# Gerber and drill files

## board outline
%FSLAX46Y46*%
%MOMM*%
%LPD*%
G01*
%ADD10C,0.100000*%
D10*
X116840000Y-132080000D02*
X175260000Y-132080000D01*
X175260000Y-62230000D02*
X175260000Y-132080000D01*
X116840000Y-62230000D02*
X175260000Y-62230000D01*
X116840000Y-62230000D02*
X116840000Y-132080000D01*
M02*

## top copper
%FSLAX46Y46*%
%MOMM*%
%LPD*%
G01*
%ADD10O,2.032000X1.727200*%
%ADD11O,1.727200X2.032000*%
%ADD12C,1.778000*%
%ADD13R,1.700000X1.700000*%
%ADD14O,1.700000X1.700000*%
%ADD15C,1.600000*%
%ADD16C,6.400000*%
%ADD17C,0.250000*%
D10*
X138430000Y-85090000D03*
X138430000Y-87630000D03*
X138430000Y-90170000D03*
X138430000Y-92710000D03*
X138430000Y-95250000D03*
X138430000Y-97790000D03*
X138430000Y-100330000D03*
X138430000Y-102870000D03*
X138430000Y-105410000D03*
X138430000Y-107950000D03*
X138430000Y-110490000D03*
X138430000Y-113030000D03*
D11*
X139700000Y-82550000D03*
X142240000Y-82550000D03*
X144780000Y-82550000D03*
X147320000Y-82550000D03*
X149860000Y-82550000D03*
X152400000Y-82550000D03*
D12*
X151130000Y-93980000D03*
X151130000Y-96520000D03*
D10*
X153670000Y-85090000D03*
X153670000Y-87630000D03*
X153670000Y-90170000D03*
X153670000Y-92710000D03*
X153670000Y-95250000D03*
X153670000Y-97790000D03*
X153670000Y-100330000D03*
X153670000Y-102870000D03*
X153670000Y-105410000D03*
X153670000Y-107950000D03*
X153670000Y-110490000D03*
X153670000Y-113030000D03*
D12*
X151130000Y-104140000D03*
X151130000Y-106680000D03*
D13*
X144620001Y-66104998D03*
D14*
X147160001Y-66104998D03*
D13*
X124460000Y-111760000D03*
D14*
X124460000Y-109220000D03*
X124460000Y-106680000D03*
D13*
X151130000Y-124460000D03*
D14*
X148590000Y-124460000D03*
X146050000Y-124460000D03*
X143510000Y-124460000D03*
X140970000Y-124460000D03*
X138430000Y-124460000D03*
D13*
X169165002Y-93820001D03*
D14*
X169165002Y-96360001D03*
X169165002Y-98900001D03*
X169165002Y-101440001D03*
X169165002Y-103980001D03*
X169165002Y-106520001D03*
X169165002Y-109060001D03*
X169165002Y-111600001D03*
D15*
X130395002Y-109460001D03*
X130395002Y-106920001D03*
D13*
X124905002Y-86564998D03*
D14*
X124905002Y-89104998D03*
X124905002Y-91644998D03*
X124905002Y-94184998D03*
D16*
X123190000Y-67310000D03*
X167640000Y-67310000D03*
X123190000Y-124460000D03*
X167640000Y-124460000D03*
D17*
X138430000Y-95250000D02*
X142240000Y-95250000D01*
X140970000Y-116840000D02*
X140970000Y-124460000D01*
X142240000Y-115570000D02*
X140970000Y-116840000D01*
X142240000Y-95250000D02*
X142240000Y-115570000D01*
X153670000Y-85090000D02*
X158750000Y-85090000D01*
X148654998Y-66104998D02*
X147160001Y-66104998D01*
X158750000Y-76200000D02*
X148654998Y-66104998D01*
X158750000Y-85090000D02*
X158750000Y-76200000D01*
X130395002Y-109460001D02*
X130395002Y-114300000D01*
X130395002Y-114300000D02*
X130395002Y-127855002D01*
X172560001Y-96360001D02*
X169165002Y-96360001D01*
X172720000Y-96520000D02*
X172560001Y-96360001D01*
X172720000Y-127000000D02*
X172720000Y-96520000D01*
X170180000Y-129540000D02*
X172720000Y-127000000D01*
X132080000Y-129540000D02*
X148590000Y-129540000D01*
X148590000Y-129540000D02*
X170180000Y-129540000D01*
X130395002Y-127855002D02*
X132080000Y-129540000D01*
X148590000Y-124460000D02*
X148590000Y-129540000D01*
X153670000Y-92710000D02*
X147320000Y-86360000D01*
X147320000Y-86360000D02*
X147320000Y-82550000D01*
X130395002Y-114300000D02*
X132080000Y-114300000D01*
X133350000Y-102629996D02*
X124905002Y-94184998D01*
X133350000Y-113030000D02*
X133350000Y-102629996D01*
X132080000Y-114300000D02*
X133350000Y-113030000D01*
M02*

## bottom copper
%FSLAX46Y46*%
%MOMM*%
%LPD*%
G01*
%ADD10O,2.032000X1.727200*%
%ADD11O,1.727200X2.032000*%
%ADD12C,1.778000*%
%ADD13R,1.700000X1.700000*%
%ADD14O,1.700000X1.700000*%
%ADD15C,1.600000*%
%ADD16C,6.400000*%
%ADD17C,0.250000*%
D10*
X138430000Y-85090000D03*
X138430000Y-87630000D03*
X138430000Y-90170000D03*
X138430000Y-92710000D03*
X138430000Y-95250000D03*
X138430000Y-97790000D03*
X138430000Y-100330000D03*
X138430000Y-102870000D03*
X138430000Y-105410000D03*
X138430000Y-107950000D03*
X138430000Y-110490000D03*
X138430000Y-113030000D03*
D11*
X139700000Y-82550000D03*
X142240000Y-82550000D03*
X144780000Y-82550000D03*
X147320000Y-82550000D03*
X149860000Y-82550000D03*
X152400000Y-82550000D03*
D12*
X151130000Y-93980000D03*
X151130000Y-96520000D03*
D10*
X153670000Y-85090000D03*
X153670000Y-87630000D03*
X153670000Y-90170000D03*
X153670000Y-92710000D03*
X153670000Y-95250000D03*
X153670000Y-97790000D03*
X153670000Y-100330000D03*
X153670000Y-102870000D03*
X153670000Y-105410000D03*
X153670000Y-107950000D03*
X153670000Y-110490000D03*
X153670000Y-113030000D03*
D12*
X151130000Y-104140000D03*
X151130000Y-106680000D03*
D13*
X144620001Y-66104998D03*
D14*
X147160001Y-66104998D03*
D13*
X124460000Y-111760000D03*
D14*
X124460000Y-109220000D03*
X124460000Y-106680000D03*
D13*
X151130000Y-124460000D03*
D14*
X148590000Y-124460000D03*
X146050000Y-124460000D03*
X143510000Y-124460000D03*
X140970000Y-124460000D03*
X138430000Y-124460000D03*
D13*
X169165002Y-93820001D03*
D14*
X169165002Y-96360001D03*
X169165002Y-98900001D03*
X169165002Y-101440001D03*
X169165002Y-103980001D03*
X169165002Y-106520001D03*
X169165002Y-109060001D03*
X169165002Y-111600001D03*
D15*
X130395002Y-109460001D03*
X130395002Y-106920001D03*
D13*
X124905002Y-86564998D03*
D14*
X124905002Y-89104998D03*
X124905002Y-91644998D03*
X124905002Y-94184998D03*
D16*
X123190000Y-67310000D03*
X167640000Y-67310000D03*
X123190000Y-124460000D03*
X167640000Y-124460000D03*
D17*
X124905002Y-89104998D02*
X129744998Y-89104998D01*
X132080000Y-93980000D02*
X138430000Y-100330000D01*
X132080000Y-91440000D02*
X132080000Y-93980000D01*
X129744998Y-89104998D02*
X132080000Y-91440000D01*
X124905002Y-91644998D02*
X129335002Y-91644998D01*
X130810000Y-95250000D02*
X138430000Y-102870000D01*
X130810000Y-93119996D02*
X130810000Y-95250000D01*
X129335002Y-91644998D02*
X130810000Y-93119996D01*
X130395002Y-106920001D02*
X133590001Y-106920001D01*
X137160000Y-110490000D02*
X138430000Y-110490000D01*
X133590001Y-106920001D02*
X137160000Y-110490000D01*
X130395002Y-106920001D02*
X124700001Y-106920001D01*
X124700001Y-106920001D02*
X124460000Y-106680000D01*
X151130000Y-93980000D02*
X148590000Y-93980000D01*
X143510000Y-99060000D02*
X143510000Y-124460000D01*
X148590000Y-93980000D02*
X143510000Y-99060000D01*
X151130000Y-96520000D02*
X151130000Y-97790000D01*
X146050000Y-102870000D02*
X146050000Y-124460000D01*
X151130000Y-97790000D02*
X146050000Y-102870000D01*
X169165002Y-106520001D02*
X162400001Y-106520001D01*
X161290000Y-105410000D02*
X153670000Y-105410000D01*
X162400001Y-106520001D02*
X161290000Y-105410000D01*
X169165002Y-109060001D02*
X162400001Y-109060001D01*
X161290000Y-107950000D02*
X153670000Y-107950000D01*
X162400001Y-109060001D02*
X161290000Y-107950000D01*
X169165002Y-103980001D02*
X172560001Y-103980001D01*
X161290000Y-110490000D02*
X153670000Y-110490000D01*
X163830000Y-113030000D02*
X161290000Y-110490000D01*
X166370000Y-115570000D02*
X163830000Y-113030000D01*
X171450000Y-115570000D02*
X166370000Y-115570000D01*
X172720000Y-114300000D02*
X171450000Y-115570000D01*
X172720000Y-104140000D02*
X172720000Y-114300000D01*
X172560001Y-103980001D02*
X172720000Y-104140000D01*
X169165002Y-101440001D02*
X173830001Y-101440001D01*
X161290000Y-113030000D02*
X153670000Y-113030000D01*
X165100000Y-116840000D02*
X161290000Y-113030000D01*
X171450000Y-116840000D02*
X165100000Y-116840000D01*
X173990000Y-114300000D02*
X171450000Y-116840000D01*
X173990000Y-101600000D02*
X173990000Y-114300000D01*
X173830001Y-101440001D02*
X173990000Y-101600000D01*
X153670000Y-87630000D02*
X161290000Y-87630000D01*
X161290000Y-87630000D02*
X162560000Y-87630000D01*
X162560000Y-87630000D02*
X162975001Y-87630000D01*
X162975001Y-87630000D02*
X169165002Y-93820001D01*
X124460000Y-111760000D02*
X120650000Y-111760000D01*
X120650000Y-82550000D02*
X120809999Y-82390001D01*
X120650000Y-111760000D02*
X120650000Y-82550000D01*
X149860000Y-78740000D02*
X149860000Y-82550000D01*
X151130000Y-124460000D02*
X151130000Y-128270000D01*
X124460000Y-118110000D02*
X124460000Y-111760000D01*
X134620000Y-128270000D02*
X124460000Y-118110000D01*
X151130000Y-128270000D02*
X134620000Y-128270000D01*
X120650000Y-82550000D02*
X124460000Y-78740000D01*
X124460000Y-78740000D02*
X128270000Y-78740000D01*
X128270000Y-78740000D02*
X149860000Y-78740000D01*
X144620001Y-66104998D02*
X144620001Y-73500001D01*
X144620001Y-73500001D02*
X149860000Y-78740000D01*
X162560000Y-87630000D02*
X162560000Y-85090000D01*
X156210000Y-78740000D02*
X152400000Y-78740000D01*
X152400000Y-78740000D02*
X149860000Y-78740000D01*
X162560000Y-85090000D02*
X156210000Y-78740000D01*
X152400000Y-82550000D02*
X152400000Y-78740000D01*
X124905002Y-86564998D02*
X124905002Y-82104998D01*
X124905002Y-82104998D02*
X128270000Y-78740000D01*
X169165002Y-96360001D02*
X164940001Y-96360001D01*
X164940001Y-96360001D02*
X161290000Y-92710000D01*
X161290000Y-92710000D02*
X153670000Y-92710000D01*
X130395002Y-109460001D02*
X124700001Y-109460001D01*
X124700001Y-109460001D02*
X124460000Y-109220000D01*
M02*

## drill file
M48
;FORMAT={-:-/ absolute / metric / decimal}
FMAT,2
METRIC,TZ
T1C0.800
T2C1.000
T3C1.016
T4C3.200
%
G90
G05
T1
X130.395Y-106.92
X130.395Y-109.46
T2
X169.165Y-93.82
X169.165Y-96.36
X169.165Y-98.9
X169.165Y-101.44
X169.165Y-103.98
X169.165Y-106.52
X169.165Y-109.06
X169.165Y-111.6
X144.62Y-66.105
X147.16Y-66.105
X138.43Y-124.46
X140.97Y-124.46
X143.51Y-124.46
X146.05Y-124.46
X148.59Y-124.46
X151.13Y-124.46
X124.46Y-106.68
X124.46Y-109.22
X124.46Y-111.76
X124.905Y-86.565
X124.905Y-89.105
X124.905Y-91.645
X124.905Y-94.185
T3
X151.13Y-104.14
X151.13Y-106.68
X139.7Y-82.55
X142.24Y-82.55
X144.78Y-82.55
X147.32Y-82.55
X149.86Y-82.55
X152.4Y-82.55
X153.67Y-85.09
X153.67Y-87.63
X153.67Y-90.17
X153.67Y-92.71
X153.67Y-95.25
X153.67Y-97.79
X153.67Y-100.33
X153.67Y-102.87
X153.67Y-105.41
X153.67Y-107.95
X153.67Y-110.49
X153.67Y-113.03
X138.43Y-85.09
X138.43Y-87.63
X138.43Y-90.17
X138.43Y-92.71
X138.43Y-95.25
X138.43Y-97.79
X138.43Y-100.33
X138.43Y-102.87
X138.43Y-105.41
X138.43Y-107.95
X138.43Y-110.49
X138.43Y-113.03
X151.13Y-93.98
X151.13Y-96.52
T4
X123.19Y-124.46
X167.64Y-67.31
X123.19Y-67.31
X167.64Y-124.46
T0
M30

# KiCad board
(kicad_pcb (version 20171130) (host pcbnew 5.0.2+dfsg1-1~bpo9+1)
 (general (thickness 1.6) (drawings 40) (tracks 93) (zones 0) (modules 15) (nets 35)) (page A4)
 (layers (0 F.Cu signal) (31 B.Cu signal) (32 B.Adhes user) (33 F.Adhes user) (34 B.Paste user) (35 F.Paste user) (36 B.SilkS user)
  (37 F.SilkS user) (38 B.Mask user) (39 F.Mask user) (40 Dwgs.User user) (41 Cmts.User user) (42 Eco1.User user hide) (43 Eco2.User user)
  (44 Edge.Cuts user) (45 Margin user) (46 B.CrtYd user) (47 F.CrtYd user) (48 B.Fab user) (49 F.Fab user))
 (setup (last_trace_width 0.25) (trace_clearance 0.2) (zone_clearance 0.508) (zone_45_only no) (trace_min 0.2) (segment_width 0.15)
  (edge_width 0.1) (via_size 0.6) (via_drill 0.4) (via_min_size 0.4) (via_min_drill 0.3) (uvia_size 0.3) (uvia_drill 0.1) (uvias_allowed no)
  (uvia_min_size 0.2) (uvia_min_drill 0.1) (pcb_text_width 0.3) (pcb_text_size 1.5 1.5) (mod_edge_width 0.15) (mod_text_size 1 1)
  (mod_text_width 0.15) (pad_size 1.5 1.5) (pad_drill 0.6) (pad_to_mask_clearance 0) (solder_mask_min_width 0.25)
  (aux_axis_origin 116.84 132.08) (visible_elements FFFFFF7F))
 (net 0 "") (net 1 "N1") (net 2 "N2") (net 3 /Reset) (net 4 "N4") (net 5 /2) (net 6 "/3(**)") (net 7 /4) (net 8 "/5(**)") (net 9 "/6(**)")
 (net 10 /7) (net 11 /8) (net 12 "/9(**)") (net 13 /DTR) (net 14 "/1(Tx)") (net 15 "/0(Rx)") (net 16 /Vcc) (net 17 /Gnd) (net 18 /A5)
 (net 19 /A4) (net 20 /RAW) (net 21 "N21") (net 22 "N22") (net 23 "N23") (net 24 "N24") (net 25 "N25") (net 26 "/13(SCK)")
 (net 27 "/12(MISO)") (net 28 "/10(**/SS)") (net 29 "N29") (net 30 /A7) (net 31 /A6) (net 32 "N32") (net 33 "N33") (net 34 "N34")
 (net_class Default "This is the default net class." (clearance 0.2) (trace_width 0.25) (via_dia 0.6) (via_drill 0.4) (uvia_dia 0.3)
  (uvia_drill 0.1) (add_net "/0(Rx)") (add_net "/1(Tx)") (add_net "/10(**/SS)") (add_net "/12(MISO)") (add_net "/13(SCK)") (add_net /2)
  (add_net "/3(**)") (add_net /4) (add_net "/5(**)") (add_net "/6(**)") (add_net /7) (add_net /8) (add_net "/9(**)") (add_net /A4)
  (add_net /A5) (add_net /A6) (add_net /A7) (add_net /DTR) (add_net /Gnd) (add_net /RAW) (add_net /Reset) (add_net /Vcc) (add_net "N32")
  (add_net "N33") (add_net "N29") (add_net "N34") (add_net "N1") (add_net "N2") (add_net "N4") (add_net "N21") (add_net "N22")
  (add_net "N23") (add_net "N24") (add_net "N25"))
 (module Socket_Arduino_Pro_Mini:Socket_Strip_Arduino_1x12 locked (layer F.Cu) (at 138.43 85.09 270)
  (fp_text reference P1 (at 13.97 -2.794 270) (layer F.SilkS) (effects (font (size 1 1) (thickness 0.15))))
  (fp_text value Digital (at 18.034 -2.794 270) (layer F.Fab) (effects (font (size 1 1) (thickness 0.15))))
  (pad 1 thru_hole oval (at 0 0 270) (size 1.7272 2.032) (drill 1.016) (layers *.Cu *.Mask F.SilkS) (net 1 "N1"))
  (pad 2 thru_hole oval (at 2.54 0 270) (size 1.7272 2.032) (drill 1.016) (layers *.Cu *.Mask F.SilkS) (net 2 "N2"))
  (pad 3 thru_hole oval (at 5.08 0 270) (size 1.7272 2.032) (drill 1.016) (layers *.Cu *.Mask F.SilkS) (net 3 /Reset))
  (pad 4 thru_hole oval (at 7.62 0 270) (size 1.7272 2.032) (drill 1.016) (layers *.Cu *.Mask F.SilkS) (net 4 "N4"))
  (pad 5 thru_hole oval (at 10.16 0 270) (size 1.7272 2.032) (drill 1.016) (layers *.Cu *.Mask F.SilkS) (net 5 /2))
  (pad 6 thru_hole oval (at 12.7 0 270) (size 1.7272 2.032) (drill 1.016) (layers *.Cu *.Mask F.SilkS) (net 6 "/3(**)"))
  (pad 7 thru_hole oval (at 15.24 0 270) (size 1.7272 2.032) (drill 1.016) (layers *.Cu *.Mask F.SilkS) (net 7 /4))
  (pad 8 thru_hole oval (at 17.78 0 270) (size 1.7272 2.032) (drill 1.016) (layers *.Cu *.Mask F.SilkS) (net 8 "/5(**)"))
  (pad 9 thru_hole oval (at 20.32 0 270) (size 1.7272 2.032) (drill 1.016) (layers *.Cu *.Mask F.SilkS) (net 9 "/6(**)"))
  (pad 10 thru_hole oval (at 22.86 0 270) (size 1.7272 2.032) (drill 1.016) (layers *.Cu *.Mask F.SilkS) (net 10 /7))
  (pad 11 thru_hole oval (at 25.4 0 270) (size 1.7272 2.032) (drill 1.016) (layers *.Cu *.Mask F.SilkS) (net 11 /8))
  (pad 12 thru_hole oval (at 27.94 0 270) (size 1.7272 2.032) (drill 1.016) (layers *.Cu *.Mask F.SilkS) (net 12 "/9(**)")))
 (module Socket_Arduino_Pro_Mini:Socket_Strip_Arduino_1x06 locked (layer F.Cu) (at 139.7 82.55)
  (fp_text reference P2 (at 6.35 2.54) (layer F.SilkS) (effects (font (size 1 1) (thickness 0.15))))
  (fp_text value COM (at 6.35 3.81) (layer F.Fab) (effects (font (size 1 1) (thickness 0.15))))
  (pad 1 thru_hole oval (at 0 0) (size 1.7272 2.032) (drill 1.016) (layers *.Cu *.Mask F.SilkS) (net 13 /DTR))
  (pad 2 thru_hole oval (at 2.54 0) (size 1.7272 2.032) (drill 1.016) (layers *.Cu *.Mask F.SilkS) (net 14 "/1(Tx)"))
  (pad 3 thru_hole oval (at 5.08 0) (size 1.7272 2.032) (drill 1.016) (layers *.Cu *.Mask F.SilkS) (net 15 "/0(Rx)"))
  (pad 4 thru_hole oval (at 7.62 0) (size 1.7272 2.032) (drill 1.016) (layers *.Cu *.Mask F.SilkS) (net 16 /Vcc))
  (pad 5 thru_hole oval (at 10.16 0) (size 1.7272 2.032) (drill 1.016) (layers *.Cu *.Mask F.SilkS) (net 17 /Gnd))
  (pad 6 thru_hole oval (at 12.7 0) (size 1.7272 2.032) (drill 1.016) (layers *.Cu *.Mask F.SilkS) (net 17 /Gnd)))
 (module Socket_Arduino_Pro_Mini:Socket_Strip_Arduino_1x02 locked (layer F.Cu) (at 151.13 93.98 270)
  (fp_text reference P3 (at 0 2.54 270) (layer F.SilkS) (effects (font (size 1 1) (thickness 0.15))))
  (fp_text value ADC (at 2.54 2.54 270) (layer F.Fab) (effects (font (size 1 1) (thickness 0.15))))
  (pad 1 thru_hole circle (at 0 0 270) (size 1.778 1.778) (drill 1.016) (layers *.Cu *.Mask F.SilkS) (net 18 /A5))
  (pad 2 thru_hole circle (at 2.54 0 270) (size 1.778 1.778) (drill 1.016) (layers *.Cu *.Mask F.SilkS) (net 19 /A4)))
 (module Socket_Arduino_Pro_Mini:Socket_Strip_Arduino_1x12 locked (layer F.Cu) (at 153.67 85.09 270)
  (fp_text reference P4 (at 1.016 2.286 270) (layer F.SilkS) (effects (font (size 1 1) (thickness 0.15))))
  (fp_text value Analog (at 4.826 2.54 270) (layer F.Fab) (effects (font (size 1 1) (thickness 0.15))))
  (pad 1 thru_hole oval (at 0 0 270) (size 1.7272 2.032) (drill 1.016) (layers *.Cu *.Mask F.SilkS) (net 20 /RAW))
  (pad 2 thru_hole oval (at 2.54 0 270) (size 1.7272 2.032) (drill 1.016) (layers *.Cu *.Mask F.SilkS) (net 17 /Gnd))
  (pad 3 thru_hole oval (at 5.08 0 270) (size 1.7272 2.032) (drill 1.016) (layers *.Cu *.Mask F.SilkS) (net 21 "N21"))
  (pad 4 thru_hole oval (at 7.62 0 270) (size 1.7272 2.032) (drill 1.016) (layers *.Cu *.Mask F.SilkS) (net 16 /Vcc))
  (pad 5 thru_hole oval (at 10.16 0 270) (size 1.7272 2.032) (drill 1.016) (layers *.Cu *.Mask F.SilkS) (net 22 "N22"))
  (pad 6 thru_hole oval (at 12.7 0 270) (size 1.7272 2.032) (drill 1.016) (layers *.Cu *.Mask F.SilkS) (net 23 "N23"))
  (pad 7 thru_hole oval (at 15.24 0 270) (size 1.7272 2.032) (drill 1.016) (layers *.Cu *.Mask F.SilkS) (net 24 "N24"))
  (pad 8 thru_hole oval (at 17.78 0 270) (size 1.7272 2.032) (drill 1.016) (layers *.Cu *.Mask F.SilkS) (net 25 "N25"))
  (pad 9 thru_hole oval (at 20.32 0 270) (size 1.7272 2.032) (drill 1.016) (layers *.Cu *.Mask F.SilkS) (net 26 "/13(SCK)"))
  (pad 10 thru_hole oval (at 22.86 0 270) (size 1.7272 2.032) (drill 1.016) (layers *.Cu *.Mask F.SilkS) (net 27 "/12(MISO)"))
  (pad 11 thru_hole oval (at 25.4 0 270) (size 1.7272 2.032) (drill 1.016) (layers *.Cu *.Mask F.SilkS) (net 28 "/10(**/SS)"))
  (pad 12 thru_hole oval (at 27.94 0 270) (size 1.7272 2.032) (drill 1.016) (layers *.Cu *.Mask F.SilkS) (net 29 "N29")))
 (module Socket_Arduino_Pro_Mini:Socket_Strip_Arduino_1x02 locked (layer F.Cu) (at 151.13 104.14 270)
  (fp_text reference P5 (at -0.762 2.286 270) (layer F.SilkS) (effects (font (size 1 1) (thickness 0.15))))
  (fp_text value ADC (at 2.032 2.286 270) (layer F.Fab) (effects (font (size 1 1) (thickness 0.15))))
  (pad 1 thru_hole circle (at 0 0 270) (size 1.778 1.778) (drill 1.016) (layers *.Cu *.Mask F.SilkS) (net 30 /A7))
  (pad 2 thru_hole circle (at 2.54 0 270) (size 1.778 1.778) (drill 1.016) (layers *.Cu *.Mask F.SilkS) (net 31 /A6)))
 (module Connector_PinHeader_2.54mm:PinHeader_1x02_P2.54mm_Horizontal (layer F.Cu) (at 144.620001 66.104998 90)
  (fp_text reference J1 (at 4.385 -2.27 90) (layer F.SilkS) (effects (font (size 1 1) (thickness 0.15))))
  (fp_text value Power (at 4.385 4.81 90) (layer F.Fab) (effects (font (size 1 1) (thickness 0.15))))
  (pad 1 thru_hole rect (at 0 0 90) (size 1.7 1.7) (drill 1) (layers *.Cu *.Mask) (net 17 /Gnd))
  (pad 2 thru_hole oval (at 0 2.54 90) (size 1.7 1.7) (drill 1) (layers *.Cu *.Mask) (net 20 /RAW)))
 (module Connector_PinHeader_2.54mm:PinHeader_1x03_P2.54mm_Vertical (layer F.Cu) (at 124.46 111.76 180)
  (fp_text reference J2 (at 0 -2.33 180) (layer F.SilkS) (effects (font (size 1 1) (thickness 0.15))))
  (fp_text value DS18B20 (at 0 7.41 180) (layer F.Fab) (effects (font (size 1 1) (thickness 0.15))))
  (pad 1 thru_hole rect (at 0 0 180) (size 1.7 1.7) (drill 1) (layers *.Cu *.Mask) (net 17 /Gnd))
  (pad 2 thru_hole oval (at 0 2.54 180) (size 1.7 1.7) (drill 1) (layers *.Cu *.Mask) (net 16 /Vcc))
  (pad 3 thru_hole oval (at 0 5.08 180) (size 1.7 1.7) (drill 1) (layers *.Cu *.Mask) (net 11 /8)))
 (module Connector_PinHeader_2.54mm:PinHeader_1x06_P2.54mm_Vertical (layer F.Cu) (at 151.13 124.46 270)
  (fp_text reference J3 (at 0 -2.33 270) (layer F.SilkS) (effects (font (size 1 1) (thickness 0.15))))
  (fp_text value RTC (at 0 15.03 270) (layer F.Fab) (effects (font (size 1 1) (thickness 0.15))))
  (pad 1 thru_hole rect (at 0 0 270) (size 1.7 1.7) (drill 1) (layers *.Cu *.Mask) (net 17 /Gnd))
  (pad 2 thru_hole oval (at 0 2.54 270) (size 1.7 1.7) (drill 1) (layers *.Cu *.Mask) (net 16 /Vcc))
  (pad 3 thru_hole oval (at 0 5.08 270) (size 1.7 1.7) (drill 1) (layers *.Cu *.Mask) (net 19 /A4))
  (pad 4 thru_hole oval (at 0 7.62 270) (size 1.7 1.7) (drill 1) (layers *.Cu *.Mask) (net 18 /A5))
  (pad 5 thru_hole oval (at 0 10.16 270) (size 1.7 1.7) (drill 1) (layers *.Cu *.Mask) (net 5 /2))
  (pad 6 thru_hole oval (at 0 12.7 270) (size 1.7 1.7) (drill 1) (layers *.Cu *.Mask) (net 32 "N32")))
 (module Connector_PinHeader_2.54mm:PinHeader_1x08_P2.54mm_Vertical (layer F.Cu) (at 169.165002 93.820001)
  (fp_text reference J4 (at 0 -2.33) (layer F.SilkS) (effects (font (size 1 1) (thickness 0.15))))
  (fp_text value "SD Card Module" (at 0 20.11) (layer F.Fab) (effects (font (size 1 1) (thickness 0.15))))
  (pad 1 thru_hole rect (at 0 0) (size 1.7 1.7) (drill 1) (layers *.Cu *.Mask) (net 17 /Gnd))
  (pad 2 thru_hole oval (at 0 2.54) (size 1.7 1.7) (drill 1) (layers *.Cu *.Mask) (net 16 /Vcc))
  (pad 3 thru_hole oval (at 0 5.08) (size 1.7 1.7) (drill 1) (layers *.Cu *.Mask) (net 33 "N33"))
  (pad 4 thru_hole oval (at 0 7.62) (size 1.7 1.7) (drill 1) (layers *.Cu *.Mask) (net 29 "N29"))
  (pad 5 thru_hole oval (at 0 10.16) (size 1.7 1.7) (drill 1) (layers *.Cu *.Mask) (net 28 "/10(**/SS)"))
  (pad 6 thru_hole oval (at 0 12.7) (size 1.7 1.7) (drill 1) (layers *.Cu *.Mask) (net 26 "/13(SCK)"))
  (pad 7 thru_hole oval (at 0 15.24) (size 1.7 1.7) (drill 1) (layers *.Cu *.Mask) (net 27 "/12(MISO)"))
  (pad 8 thru_hole oval (at 0 17.78) (size 1.7 1.7) (drill 1) (layers *.Cu *.Mask) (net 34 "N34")))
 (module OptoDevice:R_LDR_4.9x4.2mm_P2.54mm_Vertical (layer F.Cu) (at 130.395002 109.460001 90)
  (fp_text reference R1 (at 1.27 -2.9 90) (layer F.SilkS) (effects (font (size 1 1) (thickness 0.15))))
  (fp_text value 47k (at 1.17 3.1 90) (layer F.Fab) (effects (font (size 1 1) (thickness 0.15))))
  (pad 1 thru_hole circle (at 0 0 90) (size 1.6 1.6) (drill 0.8) (layers *.Cu *.Mask) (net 16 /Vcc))
  (pad 2 thru_hole circle (at 2.54 0 90) (size 1.6 1.6) (drill 0.8) (layers *.Cu *.Mask) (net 11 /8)))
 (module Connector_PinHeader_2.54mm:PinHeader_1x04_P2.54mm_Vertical (layer F.Cu) (at 124.905002 86.564998)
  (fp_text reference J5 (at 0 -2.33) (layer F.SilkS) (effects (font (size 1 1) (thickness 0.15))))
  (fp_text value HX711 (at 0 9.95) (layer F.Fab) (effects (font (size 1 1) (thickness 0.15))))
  (pad 1 thru_hole rect (at 0 0) (size 1.7 1.7) (drill 1) (layers *.Cu *.Mask) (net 17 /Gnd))
  (pad 2 thru_hole oval (at 0 2.54) (size 1.7 1.7) (drill 1) (layers *.Cu *.Mask) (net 7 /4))
  (pad 3 thru_hole oval (at 0 5.08) (size 1.7 1.7) (drill 1) (layers *.Cu *.Mask) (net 8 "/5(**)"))
  (pad 4 thru_hole oval (at 0 7.62) (size 1.7 1.7) (drill 1) (layers *.Cu *.Mask) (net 16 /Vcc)))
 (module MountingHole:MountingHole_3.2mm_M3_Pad (layer F.Cu) (at 123.19 67.31)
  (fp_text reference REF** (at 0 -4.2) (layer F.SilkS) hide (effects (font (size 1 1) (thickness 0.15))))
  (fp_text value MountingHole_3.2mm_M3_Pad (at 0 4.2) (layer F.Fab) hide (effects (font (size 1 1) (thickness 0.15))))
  (pad 1 thru_hole circle (at 0 0) (size 6.4 6.4) (drill 3.2) (layers *.Cu *.Mask)))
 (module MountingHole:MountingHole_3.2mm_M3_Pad (layer F.Cu) (at 167.64 67.31)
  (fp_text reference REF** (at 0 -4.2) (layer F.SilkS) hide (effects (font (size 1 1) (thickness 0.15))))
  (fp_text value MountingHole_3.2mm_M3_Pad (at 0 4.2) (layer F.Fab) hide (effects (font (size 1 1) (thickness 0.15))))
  (pad 1 thru_hole circle (at 0 0) (size 6.4 6.4) (drill 3.2) (layers *.Cu *.Mask)))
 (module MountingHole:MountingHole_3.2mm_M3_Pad (layer F.Cu) (at 123.19 124.46)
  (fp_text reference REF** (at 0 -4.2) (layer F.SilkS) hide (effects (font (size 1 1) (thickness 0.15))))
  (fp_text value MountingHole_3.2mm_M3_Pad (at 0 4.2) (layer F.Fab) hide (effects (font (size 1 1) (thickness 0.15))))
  (pad 1 thru_hole circle (at 0 0) (size 6.4 6.4) (drill 3.2) (layers *.Cu *.Mask)))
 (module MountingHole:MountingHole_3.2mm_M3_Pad (layer F.Cu) (at 167.64 124.46)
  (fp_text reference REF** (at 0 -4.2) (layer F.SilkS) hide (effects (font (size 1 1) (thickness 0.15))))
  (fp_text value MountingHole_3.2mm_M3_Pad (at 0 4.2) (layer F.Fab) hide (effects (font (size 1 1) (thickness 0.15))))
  (pad 1 thru_hole circle (at 0 0) (size 6.4 6.4) (drill 3.2) (layers *.Cu *.Mask)))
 (gr_line (start 116.84 132.08) (end 175.26 132.08) (angle 90) (layer Edge.Cuts) (width 0.1))
 (gr_line (start 175.26 62.23) (end 175.26 132.08) (angle 90) (layer Edge.Cuts) (width 0.1))
 (gr_line (start 116.84 62.23) (end 175.26 62.23) (angle 90) (layer Edge.Cuts) (width 0.1))
 (gr_line (start 116.84 62.23) (end 116.84 132.08) (angle 90) (layer Edge.Cuts) (width 0.1))
 (segment (start 138.43 95.25) (end 142.24 95.25) (width 0.25) (layer F.Cu) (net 5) (status 400010))
 (segment (start 140.97 116.84) (end 140.97 124.46) (width 0.25) (layer F.Cu) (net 5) (status 800020))
 (segment (start 142.24 115.57) (end 140.97 116.84) (width 0.25) (layer F.Cu) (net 5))
 (segment (start 142.24 95.25) (end 142.24 115.57) (width 0.25) (layer F.Cu) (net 5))
 (segment (start 124.905002 89.104998) (end 129.744998 89.104998) (width 0.25) (layer B.Cu) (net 7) (status 400000))
 (segment (start 132.08 93.98) (end 138.43 100.33) (width 0.25) (layer B.Cu) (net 7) (status 800000))
 (segment (start 132.08 91.44) (end 132.08 93.98) (width 0.25) (layer B.Cu) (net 7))
 (segment (start 129.744998 89.104998) (end 132.08 91.44) (width 0.25) (layer B.Cu) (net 7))
 (segment (start 124.905002 91.644998) (end 129.335002 91.644998) (width 0.25) (layer B.Cu) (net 8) (status 400000))
 (segment (start 130.81 95.25) (end 138.43 102.87) (width 0.25) (layer B.Cu) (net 8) (status 800000))
 (segment (start 130.81 93.119996) (end 130.81 95.25) (width 0.25) (layer B.Cu) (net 8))
 (segment (start 129.335002 91.644998) (end 130.81 93.119996) (width 0.25) (layer B.Cu) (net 8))
 (segment (start 130.395002 106.920001) (end 133.590001 106.920001) (width 0.25) (layer B.Cu) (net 11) (status 400010))
 (segment (start 137.16 110.49) (end 138.43 110.49) (width 0.25) (layer B.Cu) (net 11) (status 800020))
 (segment (start 133.590001 106.920001) (end 137.16 110.49) (width 0.25) (layer B.Cu) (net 11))
 (segment (start 130.395002 106.920001) (end 124.700001 106.920001) (width 0.25) (layer B.Cu) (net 11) (status C00030))
 (segment (start 124.700001 106.920001) (end 124.46 106.68) (width 0.25) (layer B.Cu) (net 11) (status C00030))
 (segment (start 151.13 93.98) (end 148.59 93.98) (width 0.25) (layer B.Cu) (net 18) (status 400010))
 (segment (start 143.51 99.06) (end 143.51 124.46) (width 0.25) (layer B.Cu) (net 18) (status 800020))
 (segment (start 148.59 93.98) (end 143.51 99.06) (width 0.25) (layer B.Cu) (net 18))
 (segment (start 151.13 96.52) (end 151.13 97.79) (width 0.25) (layer B.Cu) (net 19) (status 400010))
 (segment (start 146.05 102.87) (end 146.05 124.46) (width 0.25) (layer B.Cu) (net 19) (status 800020))
 (segment (start 151.13 97.79) (end 146.05 102.87) (width 0.25) (layer B.Cu) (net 19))
 (segment (start 153.67 85.09) (end 158.75 85.09) (width 0.25) (layer F.Cu) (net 20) (status 400010))
 (segment (start 148.654998 66.104998) (end 147.160001 66.104998) (width 0.25) (layer F.Cu) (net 20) (status 800020))
 (segment (start 158.75 76.2) (end 148.654998 66.104998) (width 0.25) (layer F.Cu) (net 20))
 (segment (start 158.75 85.09) (end 158.75 76.2) (width 0.25) (layer F.Cu) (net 20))
 (segment (start 169.165002 106.520001) (end 162.400001 106.520001) (width 0.25) (layer B.Cu) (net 26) (status 400000))
 (segment (start 161.29 105.41) (end 153.67 105.41) (width 0.25) (layer B.Cu) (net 26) (status 800000))
 (segment (start 162.400001 106.520001) (end 161.29 105.41) (width 0.25) (layer B.Cu) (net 26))
 (segment (start 169.165002 109.060001) (end 162.400001 109.060001) (width 0.25) (layer B.Cu) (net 27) (status 400000))
 (segment (start 161.29 107.95) (end 153.67 107.95) (width 0.25) (layer B.Cu) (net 27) (status 800000))
 (segment (start 162.400001 109.060001) (end 161.29 107.95) (width 0.25) (layer B.Cu) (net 27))
 (segment (start 169.165002 103.980001) (end 172.560001 103.980001) (width 0.25) (layer B.Cu) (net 28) (status 400000))
 (segment (start 161.29 110.49) (end 153.67 110.49) (width 0.25) (layer B.Cu) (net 28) (status 800000))
 (segment (start 163.83 113.03) (end 161.29 110.49) (width 0.25) (layer B.Cu) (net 28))
 (segment (start 166.37 115.57) (end 163.83 113.03) (width 0.25) (layer B.Cu) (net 28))
 (segment (start 171.45 115.57) (end 166.37 115.57) (width 0.25) (layer B.Cu) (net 28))
 (segment (start 172.72 114.3) (end 171.45 115.57) (width 0.25) (layer B.Cu) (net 28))
 (segment (start 172.72 104.14) (end 172.72 114.3) (width 0.25) (layer B.Cu) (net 28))
 (segment (start 172.560001 103.980001) (end 172.72 104.14) (width 0.25) (layer B.Cu) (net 28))
 (segment (start 169.165002 101.440001) (end 173.830001 101.440001) (width 0.25) (layer B.Cu) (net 29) (status 400000))
 (segment (start 161.29 113.03) (end 153.67 113.03) (width 0.25) (layer B.Cu) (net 29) (status 800000))
 (segment (start 165.1 116.84) (end 161.29 113.03) (width 0.25) (layer B.Cu) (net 29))
 (segment (start 171.45 116.84) (end 165.1 116.84) (width 0.25) (layer B.Cu) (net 29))
 (segment (start 173.99 114.3) (end 171.45 116.84) (width 0.25) (layer B.Cu) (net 29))
 (segment (start 173.99 101.6) (end 173.99 114.3) (width 0.25) (layer B.Cu) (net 29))
 (segment (start 173.830001 101.440001) (end 173.99 101.6) (width 0.25) (layer B.Cu) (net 29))
 (segment (start 153.67 87.63) (end 161.29 87.63) (width 0.25) (layer B.Cu) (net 17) (status 400010))
 (segment (start 161.29 87.63) (end 162.56 87.63) (width 0.25) (layer B.Cu) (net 17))
 (segment (start 162.56 87.63) (end 162.975001 87.63) (width 0.25) (layer B.Cu) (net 17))
 (segment (start 162.975001 87.63) (end 169.165002 93.820001) (width 0.25) (layer B.Cu) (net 17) (status 800020))
 (segment (start 124.46 111.76) (end 120.65 111.76) (width 0.25) (layer B.Cu) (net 17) (status 400010))
 (segment (start 120.65 82.55) (end 120.809999 82.390001) (width 0.25) (layer B.Cu) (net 17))
 (segment (start 120.65 111.76) (end 120.65 82.55) (width 0.25) (layer B.Cu) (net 17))
 (segment (start 149.86 78.74) (end 149.86 82.55) (width 0.25) (layer B.Cu) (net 17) (status 800020))
 (segment (start 151.13 124.46) (end 151.13 128.27) (width 0.25) (layer B.Cu) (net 17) (status 400010))
 (segment (start 124.46 118.11) (end 124.46 111.76) (width 0.25) (layer B.Cu) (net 17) (status 800020))
 (segment (start 134.62 128.27) (end 124.46 118.11) (width 0.25) (layer B.Cu) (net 17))
 (segment (start 151.13 128.27) (end 134.62 128.27) (width 0.25) (layer B.Cu) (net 17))
 (segment (start 120.65 82.55) (end 124.46 78.74) (width 0.25) (layer B.Cu) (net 17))
 (segment (start 124.46 78.74) (end 128.27 78.74) (width 0.25) (layer B.Cu) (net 17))
 (segment (start 128.27 78.74) (end 149.86 78.74) (width 0.25) (layer B.Cu) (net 17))
 (segment (start 144.620001 66.104998) (end 144.620001 73.500001) (width 0.25) (layer B.Cu) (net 17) (status 400010))
 (segment (start 144.620001 73.500001) (end 149.86 78.74) (width 0.25) (layer B.Cu) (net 17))
 (segment (start 162.56 87.63) (end 162.56 85.09) (width 0.25) (layer B.Cu) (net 17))
 (segment (start 156.21 78.74) (end 152.4 78.74) (width 0.25) (layer B.Cu) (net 17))
 (segment (start 152.4 78.74) (end 149.86 78.74) (width 0.25) (layer B.Cu) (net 17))
 (segment (start 162.56 85.09) (end 156.21 78.74) (width 0.25) (layer B.Cu) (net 17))
 (segment (start 152.4 82.55) (end 152.4 78.74) (width 0.25) (layer B.Cu) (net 17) (status 400000))
 (segment (start 124.905002 86.564998) (end 124.905002 82.104998) (width 0.25) (layer B.Cu) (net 17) (status 400000))
 (segment (start 124.905002 82.104998) (end 128.27 78.74) (width 0.25) (layer B.Cu) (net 17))
 (segment (start 169.165002 96.360001) (end 164.940001 96.360001) (width 0.25) (layer B.Cu) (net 16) (status 400010))
 (segment (start 164.940001 96.360001) (end 161.29 92.71) (width 0.25) (layer B.Cu) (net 16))
 (segment (start 161.29 92.71) (end 153.67 92.71) (width 0.25) (layer B.Cu) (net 16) (status 800020))
 (segment (start 130.395002 109.460001) (end 124.700001 109.460001) (width 0.25) (layer B.Cu) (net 16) (status C00030))
 (segment (start 124.700001 109.460001) (end 124.46 109.22) (width 0.25) (layer B.Cu) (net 16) (status C00030))
 (segment (start 130.395002 109.460001) (end 130.395002 114.3) (width 0.25) (layer F.Cu) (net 16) (status 400010))
 (segment (start 130.395002 114.3) (end 130.395002 127.855002) (width 0.25) (layer F.Cu) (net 16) (status 10))
 (segment (start 172.560001 96.360001) (end 169.165002 96.360001) (width 0.25) (layer F.Cu) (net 16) (status 800020))
 (segment (start 172.72 96.52) (end 172.560001 96.360001) (width 0.25) (layer F.Cu) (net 16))
 (segment (start 172.72 127) (end 172.72 96.52) (width 0.25) (layer F.Cu) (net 16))
 (segment (start 170.18 129.54) (end 172.72 127) (width 0.25) (layer F.Cu) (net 16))
 (segment (start 132.08 129.54) (end 148.59 129.54) (width 0.25) (layer F.Cu) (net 16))
 (segment (start 148.59 129.54) (end 170.18 129.54) (width 0.25) (layer F.Cu) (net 16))
 (segment (start 130.395002 127.855002) (end 132.08 129.54) (width 0.25) (layer F.Cu) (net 16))
 (segment (start 148.59 124.46) (end 148.59 129.54) (width 0.25) (layer F.Cu) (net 16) (status 400010))
 (segment (start 153.67 92.71) (end 147.32 86.36) (width 0.25) (layer F.Cu) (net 16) (status 400000))
 (segment (start 147.32 86.36) (end 147.32 82.55) (width 0.25) (layer F.Cu) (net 16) (status 800000))
 (segment (start 130.395002 114.3) (end 132.08 114.3) (width 0.25) (layer F.Cu) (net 16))
 (segment (start 133.35 102.629996) (end 124.905002 94.184998) (width 0.25) (layer F.Cu) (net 16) (status 800000))
 (segment (start 133.35 113.03) (end 133.35 102.629996) (width 0.25) (layer F.Cu) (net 16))
 (segment (start 132.08 114.3) (end 133.35 113.03) (width 0.25) (layer F.Cu) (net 16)))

